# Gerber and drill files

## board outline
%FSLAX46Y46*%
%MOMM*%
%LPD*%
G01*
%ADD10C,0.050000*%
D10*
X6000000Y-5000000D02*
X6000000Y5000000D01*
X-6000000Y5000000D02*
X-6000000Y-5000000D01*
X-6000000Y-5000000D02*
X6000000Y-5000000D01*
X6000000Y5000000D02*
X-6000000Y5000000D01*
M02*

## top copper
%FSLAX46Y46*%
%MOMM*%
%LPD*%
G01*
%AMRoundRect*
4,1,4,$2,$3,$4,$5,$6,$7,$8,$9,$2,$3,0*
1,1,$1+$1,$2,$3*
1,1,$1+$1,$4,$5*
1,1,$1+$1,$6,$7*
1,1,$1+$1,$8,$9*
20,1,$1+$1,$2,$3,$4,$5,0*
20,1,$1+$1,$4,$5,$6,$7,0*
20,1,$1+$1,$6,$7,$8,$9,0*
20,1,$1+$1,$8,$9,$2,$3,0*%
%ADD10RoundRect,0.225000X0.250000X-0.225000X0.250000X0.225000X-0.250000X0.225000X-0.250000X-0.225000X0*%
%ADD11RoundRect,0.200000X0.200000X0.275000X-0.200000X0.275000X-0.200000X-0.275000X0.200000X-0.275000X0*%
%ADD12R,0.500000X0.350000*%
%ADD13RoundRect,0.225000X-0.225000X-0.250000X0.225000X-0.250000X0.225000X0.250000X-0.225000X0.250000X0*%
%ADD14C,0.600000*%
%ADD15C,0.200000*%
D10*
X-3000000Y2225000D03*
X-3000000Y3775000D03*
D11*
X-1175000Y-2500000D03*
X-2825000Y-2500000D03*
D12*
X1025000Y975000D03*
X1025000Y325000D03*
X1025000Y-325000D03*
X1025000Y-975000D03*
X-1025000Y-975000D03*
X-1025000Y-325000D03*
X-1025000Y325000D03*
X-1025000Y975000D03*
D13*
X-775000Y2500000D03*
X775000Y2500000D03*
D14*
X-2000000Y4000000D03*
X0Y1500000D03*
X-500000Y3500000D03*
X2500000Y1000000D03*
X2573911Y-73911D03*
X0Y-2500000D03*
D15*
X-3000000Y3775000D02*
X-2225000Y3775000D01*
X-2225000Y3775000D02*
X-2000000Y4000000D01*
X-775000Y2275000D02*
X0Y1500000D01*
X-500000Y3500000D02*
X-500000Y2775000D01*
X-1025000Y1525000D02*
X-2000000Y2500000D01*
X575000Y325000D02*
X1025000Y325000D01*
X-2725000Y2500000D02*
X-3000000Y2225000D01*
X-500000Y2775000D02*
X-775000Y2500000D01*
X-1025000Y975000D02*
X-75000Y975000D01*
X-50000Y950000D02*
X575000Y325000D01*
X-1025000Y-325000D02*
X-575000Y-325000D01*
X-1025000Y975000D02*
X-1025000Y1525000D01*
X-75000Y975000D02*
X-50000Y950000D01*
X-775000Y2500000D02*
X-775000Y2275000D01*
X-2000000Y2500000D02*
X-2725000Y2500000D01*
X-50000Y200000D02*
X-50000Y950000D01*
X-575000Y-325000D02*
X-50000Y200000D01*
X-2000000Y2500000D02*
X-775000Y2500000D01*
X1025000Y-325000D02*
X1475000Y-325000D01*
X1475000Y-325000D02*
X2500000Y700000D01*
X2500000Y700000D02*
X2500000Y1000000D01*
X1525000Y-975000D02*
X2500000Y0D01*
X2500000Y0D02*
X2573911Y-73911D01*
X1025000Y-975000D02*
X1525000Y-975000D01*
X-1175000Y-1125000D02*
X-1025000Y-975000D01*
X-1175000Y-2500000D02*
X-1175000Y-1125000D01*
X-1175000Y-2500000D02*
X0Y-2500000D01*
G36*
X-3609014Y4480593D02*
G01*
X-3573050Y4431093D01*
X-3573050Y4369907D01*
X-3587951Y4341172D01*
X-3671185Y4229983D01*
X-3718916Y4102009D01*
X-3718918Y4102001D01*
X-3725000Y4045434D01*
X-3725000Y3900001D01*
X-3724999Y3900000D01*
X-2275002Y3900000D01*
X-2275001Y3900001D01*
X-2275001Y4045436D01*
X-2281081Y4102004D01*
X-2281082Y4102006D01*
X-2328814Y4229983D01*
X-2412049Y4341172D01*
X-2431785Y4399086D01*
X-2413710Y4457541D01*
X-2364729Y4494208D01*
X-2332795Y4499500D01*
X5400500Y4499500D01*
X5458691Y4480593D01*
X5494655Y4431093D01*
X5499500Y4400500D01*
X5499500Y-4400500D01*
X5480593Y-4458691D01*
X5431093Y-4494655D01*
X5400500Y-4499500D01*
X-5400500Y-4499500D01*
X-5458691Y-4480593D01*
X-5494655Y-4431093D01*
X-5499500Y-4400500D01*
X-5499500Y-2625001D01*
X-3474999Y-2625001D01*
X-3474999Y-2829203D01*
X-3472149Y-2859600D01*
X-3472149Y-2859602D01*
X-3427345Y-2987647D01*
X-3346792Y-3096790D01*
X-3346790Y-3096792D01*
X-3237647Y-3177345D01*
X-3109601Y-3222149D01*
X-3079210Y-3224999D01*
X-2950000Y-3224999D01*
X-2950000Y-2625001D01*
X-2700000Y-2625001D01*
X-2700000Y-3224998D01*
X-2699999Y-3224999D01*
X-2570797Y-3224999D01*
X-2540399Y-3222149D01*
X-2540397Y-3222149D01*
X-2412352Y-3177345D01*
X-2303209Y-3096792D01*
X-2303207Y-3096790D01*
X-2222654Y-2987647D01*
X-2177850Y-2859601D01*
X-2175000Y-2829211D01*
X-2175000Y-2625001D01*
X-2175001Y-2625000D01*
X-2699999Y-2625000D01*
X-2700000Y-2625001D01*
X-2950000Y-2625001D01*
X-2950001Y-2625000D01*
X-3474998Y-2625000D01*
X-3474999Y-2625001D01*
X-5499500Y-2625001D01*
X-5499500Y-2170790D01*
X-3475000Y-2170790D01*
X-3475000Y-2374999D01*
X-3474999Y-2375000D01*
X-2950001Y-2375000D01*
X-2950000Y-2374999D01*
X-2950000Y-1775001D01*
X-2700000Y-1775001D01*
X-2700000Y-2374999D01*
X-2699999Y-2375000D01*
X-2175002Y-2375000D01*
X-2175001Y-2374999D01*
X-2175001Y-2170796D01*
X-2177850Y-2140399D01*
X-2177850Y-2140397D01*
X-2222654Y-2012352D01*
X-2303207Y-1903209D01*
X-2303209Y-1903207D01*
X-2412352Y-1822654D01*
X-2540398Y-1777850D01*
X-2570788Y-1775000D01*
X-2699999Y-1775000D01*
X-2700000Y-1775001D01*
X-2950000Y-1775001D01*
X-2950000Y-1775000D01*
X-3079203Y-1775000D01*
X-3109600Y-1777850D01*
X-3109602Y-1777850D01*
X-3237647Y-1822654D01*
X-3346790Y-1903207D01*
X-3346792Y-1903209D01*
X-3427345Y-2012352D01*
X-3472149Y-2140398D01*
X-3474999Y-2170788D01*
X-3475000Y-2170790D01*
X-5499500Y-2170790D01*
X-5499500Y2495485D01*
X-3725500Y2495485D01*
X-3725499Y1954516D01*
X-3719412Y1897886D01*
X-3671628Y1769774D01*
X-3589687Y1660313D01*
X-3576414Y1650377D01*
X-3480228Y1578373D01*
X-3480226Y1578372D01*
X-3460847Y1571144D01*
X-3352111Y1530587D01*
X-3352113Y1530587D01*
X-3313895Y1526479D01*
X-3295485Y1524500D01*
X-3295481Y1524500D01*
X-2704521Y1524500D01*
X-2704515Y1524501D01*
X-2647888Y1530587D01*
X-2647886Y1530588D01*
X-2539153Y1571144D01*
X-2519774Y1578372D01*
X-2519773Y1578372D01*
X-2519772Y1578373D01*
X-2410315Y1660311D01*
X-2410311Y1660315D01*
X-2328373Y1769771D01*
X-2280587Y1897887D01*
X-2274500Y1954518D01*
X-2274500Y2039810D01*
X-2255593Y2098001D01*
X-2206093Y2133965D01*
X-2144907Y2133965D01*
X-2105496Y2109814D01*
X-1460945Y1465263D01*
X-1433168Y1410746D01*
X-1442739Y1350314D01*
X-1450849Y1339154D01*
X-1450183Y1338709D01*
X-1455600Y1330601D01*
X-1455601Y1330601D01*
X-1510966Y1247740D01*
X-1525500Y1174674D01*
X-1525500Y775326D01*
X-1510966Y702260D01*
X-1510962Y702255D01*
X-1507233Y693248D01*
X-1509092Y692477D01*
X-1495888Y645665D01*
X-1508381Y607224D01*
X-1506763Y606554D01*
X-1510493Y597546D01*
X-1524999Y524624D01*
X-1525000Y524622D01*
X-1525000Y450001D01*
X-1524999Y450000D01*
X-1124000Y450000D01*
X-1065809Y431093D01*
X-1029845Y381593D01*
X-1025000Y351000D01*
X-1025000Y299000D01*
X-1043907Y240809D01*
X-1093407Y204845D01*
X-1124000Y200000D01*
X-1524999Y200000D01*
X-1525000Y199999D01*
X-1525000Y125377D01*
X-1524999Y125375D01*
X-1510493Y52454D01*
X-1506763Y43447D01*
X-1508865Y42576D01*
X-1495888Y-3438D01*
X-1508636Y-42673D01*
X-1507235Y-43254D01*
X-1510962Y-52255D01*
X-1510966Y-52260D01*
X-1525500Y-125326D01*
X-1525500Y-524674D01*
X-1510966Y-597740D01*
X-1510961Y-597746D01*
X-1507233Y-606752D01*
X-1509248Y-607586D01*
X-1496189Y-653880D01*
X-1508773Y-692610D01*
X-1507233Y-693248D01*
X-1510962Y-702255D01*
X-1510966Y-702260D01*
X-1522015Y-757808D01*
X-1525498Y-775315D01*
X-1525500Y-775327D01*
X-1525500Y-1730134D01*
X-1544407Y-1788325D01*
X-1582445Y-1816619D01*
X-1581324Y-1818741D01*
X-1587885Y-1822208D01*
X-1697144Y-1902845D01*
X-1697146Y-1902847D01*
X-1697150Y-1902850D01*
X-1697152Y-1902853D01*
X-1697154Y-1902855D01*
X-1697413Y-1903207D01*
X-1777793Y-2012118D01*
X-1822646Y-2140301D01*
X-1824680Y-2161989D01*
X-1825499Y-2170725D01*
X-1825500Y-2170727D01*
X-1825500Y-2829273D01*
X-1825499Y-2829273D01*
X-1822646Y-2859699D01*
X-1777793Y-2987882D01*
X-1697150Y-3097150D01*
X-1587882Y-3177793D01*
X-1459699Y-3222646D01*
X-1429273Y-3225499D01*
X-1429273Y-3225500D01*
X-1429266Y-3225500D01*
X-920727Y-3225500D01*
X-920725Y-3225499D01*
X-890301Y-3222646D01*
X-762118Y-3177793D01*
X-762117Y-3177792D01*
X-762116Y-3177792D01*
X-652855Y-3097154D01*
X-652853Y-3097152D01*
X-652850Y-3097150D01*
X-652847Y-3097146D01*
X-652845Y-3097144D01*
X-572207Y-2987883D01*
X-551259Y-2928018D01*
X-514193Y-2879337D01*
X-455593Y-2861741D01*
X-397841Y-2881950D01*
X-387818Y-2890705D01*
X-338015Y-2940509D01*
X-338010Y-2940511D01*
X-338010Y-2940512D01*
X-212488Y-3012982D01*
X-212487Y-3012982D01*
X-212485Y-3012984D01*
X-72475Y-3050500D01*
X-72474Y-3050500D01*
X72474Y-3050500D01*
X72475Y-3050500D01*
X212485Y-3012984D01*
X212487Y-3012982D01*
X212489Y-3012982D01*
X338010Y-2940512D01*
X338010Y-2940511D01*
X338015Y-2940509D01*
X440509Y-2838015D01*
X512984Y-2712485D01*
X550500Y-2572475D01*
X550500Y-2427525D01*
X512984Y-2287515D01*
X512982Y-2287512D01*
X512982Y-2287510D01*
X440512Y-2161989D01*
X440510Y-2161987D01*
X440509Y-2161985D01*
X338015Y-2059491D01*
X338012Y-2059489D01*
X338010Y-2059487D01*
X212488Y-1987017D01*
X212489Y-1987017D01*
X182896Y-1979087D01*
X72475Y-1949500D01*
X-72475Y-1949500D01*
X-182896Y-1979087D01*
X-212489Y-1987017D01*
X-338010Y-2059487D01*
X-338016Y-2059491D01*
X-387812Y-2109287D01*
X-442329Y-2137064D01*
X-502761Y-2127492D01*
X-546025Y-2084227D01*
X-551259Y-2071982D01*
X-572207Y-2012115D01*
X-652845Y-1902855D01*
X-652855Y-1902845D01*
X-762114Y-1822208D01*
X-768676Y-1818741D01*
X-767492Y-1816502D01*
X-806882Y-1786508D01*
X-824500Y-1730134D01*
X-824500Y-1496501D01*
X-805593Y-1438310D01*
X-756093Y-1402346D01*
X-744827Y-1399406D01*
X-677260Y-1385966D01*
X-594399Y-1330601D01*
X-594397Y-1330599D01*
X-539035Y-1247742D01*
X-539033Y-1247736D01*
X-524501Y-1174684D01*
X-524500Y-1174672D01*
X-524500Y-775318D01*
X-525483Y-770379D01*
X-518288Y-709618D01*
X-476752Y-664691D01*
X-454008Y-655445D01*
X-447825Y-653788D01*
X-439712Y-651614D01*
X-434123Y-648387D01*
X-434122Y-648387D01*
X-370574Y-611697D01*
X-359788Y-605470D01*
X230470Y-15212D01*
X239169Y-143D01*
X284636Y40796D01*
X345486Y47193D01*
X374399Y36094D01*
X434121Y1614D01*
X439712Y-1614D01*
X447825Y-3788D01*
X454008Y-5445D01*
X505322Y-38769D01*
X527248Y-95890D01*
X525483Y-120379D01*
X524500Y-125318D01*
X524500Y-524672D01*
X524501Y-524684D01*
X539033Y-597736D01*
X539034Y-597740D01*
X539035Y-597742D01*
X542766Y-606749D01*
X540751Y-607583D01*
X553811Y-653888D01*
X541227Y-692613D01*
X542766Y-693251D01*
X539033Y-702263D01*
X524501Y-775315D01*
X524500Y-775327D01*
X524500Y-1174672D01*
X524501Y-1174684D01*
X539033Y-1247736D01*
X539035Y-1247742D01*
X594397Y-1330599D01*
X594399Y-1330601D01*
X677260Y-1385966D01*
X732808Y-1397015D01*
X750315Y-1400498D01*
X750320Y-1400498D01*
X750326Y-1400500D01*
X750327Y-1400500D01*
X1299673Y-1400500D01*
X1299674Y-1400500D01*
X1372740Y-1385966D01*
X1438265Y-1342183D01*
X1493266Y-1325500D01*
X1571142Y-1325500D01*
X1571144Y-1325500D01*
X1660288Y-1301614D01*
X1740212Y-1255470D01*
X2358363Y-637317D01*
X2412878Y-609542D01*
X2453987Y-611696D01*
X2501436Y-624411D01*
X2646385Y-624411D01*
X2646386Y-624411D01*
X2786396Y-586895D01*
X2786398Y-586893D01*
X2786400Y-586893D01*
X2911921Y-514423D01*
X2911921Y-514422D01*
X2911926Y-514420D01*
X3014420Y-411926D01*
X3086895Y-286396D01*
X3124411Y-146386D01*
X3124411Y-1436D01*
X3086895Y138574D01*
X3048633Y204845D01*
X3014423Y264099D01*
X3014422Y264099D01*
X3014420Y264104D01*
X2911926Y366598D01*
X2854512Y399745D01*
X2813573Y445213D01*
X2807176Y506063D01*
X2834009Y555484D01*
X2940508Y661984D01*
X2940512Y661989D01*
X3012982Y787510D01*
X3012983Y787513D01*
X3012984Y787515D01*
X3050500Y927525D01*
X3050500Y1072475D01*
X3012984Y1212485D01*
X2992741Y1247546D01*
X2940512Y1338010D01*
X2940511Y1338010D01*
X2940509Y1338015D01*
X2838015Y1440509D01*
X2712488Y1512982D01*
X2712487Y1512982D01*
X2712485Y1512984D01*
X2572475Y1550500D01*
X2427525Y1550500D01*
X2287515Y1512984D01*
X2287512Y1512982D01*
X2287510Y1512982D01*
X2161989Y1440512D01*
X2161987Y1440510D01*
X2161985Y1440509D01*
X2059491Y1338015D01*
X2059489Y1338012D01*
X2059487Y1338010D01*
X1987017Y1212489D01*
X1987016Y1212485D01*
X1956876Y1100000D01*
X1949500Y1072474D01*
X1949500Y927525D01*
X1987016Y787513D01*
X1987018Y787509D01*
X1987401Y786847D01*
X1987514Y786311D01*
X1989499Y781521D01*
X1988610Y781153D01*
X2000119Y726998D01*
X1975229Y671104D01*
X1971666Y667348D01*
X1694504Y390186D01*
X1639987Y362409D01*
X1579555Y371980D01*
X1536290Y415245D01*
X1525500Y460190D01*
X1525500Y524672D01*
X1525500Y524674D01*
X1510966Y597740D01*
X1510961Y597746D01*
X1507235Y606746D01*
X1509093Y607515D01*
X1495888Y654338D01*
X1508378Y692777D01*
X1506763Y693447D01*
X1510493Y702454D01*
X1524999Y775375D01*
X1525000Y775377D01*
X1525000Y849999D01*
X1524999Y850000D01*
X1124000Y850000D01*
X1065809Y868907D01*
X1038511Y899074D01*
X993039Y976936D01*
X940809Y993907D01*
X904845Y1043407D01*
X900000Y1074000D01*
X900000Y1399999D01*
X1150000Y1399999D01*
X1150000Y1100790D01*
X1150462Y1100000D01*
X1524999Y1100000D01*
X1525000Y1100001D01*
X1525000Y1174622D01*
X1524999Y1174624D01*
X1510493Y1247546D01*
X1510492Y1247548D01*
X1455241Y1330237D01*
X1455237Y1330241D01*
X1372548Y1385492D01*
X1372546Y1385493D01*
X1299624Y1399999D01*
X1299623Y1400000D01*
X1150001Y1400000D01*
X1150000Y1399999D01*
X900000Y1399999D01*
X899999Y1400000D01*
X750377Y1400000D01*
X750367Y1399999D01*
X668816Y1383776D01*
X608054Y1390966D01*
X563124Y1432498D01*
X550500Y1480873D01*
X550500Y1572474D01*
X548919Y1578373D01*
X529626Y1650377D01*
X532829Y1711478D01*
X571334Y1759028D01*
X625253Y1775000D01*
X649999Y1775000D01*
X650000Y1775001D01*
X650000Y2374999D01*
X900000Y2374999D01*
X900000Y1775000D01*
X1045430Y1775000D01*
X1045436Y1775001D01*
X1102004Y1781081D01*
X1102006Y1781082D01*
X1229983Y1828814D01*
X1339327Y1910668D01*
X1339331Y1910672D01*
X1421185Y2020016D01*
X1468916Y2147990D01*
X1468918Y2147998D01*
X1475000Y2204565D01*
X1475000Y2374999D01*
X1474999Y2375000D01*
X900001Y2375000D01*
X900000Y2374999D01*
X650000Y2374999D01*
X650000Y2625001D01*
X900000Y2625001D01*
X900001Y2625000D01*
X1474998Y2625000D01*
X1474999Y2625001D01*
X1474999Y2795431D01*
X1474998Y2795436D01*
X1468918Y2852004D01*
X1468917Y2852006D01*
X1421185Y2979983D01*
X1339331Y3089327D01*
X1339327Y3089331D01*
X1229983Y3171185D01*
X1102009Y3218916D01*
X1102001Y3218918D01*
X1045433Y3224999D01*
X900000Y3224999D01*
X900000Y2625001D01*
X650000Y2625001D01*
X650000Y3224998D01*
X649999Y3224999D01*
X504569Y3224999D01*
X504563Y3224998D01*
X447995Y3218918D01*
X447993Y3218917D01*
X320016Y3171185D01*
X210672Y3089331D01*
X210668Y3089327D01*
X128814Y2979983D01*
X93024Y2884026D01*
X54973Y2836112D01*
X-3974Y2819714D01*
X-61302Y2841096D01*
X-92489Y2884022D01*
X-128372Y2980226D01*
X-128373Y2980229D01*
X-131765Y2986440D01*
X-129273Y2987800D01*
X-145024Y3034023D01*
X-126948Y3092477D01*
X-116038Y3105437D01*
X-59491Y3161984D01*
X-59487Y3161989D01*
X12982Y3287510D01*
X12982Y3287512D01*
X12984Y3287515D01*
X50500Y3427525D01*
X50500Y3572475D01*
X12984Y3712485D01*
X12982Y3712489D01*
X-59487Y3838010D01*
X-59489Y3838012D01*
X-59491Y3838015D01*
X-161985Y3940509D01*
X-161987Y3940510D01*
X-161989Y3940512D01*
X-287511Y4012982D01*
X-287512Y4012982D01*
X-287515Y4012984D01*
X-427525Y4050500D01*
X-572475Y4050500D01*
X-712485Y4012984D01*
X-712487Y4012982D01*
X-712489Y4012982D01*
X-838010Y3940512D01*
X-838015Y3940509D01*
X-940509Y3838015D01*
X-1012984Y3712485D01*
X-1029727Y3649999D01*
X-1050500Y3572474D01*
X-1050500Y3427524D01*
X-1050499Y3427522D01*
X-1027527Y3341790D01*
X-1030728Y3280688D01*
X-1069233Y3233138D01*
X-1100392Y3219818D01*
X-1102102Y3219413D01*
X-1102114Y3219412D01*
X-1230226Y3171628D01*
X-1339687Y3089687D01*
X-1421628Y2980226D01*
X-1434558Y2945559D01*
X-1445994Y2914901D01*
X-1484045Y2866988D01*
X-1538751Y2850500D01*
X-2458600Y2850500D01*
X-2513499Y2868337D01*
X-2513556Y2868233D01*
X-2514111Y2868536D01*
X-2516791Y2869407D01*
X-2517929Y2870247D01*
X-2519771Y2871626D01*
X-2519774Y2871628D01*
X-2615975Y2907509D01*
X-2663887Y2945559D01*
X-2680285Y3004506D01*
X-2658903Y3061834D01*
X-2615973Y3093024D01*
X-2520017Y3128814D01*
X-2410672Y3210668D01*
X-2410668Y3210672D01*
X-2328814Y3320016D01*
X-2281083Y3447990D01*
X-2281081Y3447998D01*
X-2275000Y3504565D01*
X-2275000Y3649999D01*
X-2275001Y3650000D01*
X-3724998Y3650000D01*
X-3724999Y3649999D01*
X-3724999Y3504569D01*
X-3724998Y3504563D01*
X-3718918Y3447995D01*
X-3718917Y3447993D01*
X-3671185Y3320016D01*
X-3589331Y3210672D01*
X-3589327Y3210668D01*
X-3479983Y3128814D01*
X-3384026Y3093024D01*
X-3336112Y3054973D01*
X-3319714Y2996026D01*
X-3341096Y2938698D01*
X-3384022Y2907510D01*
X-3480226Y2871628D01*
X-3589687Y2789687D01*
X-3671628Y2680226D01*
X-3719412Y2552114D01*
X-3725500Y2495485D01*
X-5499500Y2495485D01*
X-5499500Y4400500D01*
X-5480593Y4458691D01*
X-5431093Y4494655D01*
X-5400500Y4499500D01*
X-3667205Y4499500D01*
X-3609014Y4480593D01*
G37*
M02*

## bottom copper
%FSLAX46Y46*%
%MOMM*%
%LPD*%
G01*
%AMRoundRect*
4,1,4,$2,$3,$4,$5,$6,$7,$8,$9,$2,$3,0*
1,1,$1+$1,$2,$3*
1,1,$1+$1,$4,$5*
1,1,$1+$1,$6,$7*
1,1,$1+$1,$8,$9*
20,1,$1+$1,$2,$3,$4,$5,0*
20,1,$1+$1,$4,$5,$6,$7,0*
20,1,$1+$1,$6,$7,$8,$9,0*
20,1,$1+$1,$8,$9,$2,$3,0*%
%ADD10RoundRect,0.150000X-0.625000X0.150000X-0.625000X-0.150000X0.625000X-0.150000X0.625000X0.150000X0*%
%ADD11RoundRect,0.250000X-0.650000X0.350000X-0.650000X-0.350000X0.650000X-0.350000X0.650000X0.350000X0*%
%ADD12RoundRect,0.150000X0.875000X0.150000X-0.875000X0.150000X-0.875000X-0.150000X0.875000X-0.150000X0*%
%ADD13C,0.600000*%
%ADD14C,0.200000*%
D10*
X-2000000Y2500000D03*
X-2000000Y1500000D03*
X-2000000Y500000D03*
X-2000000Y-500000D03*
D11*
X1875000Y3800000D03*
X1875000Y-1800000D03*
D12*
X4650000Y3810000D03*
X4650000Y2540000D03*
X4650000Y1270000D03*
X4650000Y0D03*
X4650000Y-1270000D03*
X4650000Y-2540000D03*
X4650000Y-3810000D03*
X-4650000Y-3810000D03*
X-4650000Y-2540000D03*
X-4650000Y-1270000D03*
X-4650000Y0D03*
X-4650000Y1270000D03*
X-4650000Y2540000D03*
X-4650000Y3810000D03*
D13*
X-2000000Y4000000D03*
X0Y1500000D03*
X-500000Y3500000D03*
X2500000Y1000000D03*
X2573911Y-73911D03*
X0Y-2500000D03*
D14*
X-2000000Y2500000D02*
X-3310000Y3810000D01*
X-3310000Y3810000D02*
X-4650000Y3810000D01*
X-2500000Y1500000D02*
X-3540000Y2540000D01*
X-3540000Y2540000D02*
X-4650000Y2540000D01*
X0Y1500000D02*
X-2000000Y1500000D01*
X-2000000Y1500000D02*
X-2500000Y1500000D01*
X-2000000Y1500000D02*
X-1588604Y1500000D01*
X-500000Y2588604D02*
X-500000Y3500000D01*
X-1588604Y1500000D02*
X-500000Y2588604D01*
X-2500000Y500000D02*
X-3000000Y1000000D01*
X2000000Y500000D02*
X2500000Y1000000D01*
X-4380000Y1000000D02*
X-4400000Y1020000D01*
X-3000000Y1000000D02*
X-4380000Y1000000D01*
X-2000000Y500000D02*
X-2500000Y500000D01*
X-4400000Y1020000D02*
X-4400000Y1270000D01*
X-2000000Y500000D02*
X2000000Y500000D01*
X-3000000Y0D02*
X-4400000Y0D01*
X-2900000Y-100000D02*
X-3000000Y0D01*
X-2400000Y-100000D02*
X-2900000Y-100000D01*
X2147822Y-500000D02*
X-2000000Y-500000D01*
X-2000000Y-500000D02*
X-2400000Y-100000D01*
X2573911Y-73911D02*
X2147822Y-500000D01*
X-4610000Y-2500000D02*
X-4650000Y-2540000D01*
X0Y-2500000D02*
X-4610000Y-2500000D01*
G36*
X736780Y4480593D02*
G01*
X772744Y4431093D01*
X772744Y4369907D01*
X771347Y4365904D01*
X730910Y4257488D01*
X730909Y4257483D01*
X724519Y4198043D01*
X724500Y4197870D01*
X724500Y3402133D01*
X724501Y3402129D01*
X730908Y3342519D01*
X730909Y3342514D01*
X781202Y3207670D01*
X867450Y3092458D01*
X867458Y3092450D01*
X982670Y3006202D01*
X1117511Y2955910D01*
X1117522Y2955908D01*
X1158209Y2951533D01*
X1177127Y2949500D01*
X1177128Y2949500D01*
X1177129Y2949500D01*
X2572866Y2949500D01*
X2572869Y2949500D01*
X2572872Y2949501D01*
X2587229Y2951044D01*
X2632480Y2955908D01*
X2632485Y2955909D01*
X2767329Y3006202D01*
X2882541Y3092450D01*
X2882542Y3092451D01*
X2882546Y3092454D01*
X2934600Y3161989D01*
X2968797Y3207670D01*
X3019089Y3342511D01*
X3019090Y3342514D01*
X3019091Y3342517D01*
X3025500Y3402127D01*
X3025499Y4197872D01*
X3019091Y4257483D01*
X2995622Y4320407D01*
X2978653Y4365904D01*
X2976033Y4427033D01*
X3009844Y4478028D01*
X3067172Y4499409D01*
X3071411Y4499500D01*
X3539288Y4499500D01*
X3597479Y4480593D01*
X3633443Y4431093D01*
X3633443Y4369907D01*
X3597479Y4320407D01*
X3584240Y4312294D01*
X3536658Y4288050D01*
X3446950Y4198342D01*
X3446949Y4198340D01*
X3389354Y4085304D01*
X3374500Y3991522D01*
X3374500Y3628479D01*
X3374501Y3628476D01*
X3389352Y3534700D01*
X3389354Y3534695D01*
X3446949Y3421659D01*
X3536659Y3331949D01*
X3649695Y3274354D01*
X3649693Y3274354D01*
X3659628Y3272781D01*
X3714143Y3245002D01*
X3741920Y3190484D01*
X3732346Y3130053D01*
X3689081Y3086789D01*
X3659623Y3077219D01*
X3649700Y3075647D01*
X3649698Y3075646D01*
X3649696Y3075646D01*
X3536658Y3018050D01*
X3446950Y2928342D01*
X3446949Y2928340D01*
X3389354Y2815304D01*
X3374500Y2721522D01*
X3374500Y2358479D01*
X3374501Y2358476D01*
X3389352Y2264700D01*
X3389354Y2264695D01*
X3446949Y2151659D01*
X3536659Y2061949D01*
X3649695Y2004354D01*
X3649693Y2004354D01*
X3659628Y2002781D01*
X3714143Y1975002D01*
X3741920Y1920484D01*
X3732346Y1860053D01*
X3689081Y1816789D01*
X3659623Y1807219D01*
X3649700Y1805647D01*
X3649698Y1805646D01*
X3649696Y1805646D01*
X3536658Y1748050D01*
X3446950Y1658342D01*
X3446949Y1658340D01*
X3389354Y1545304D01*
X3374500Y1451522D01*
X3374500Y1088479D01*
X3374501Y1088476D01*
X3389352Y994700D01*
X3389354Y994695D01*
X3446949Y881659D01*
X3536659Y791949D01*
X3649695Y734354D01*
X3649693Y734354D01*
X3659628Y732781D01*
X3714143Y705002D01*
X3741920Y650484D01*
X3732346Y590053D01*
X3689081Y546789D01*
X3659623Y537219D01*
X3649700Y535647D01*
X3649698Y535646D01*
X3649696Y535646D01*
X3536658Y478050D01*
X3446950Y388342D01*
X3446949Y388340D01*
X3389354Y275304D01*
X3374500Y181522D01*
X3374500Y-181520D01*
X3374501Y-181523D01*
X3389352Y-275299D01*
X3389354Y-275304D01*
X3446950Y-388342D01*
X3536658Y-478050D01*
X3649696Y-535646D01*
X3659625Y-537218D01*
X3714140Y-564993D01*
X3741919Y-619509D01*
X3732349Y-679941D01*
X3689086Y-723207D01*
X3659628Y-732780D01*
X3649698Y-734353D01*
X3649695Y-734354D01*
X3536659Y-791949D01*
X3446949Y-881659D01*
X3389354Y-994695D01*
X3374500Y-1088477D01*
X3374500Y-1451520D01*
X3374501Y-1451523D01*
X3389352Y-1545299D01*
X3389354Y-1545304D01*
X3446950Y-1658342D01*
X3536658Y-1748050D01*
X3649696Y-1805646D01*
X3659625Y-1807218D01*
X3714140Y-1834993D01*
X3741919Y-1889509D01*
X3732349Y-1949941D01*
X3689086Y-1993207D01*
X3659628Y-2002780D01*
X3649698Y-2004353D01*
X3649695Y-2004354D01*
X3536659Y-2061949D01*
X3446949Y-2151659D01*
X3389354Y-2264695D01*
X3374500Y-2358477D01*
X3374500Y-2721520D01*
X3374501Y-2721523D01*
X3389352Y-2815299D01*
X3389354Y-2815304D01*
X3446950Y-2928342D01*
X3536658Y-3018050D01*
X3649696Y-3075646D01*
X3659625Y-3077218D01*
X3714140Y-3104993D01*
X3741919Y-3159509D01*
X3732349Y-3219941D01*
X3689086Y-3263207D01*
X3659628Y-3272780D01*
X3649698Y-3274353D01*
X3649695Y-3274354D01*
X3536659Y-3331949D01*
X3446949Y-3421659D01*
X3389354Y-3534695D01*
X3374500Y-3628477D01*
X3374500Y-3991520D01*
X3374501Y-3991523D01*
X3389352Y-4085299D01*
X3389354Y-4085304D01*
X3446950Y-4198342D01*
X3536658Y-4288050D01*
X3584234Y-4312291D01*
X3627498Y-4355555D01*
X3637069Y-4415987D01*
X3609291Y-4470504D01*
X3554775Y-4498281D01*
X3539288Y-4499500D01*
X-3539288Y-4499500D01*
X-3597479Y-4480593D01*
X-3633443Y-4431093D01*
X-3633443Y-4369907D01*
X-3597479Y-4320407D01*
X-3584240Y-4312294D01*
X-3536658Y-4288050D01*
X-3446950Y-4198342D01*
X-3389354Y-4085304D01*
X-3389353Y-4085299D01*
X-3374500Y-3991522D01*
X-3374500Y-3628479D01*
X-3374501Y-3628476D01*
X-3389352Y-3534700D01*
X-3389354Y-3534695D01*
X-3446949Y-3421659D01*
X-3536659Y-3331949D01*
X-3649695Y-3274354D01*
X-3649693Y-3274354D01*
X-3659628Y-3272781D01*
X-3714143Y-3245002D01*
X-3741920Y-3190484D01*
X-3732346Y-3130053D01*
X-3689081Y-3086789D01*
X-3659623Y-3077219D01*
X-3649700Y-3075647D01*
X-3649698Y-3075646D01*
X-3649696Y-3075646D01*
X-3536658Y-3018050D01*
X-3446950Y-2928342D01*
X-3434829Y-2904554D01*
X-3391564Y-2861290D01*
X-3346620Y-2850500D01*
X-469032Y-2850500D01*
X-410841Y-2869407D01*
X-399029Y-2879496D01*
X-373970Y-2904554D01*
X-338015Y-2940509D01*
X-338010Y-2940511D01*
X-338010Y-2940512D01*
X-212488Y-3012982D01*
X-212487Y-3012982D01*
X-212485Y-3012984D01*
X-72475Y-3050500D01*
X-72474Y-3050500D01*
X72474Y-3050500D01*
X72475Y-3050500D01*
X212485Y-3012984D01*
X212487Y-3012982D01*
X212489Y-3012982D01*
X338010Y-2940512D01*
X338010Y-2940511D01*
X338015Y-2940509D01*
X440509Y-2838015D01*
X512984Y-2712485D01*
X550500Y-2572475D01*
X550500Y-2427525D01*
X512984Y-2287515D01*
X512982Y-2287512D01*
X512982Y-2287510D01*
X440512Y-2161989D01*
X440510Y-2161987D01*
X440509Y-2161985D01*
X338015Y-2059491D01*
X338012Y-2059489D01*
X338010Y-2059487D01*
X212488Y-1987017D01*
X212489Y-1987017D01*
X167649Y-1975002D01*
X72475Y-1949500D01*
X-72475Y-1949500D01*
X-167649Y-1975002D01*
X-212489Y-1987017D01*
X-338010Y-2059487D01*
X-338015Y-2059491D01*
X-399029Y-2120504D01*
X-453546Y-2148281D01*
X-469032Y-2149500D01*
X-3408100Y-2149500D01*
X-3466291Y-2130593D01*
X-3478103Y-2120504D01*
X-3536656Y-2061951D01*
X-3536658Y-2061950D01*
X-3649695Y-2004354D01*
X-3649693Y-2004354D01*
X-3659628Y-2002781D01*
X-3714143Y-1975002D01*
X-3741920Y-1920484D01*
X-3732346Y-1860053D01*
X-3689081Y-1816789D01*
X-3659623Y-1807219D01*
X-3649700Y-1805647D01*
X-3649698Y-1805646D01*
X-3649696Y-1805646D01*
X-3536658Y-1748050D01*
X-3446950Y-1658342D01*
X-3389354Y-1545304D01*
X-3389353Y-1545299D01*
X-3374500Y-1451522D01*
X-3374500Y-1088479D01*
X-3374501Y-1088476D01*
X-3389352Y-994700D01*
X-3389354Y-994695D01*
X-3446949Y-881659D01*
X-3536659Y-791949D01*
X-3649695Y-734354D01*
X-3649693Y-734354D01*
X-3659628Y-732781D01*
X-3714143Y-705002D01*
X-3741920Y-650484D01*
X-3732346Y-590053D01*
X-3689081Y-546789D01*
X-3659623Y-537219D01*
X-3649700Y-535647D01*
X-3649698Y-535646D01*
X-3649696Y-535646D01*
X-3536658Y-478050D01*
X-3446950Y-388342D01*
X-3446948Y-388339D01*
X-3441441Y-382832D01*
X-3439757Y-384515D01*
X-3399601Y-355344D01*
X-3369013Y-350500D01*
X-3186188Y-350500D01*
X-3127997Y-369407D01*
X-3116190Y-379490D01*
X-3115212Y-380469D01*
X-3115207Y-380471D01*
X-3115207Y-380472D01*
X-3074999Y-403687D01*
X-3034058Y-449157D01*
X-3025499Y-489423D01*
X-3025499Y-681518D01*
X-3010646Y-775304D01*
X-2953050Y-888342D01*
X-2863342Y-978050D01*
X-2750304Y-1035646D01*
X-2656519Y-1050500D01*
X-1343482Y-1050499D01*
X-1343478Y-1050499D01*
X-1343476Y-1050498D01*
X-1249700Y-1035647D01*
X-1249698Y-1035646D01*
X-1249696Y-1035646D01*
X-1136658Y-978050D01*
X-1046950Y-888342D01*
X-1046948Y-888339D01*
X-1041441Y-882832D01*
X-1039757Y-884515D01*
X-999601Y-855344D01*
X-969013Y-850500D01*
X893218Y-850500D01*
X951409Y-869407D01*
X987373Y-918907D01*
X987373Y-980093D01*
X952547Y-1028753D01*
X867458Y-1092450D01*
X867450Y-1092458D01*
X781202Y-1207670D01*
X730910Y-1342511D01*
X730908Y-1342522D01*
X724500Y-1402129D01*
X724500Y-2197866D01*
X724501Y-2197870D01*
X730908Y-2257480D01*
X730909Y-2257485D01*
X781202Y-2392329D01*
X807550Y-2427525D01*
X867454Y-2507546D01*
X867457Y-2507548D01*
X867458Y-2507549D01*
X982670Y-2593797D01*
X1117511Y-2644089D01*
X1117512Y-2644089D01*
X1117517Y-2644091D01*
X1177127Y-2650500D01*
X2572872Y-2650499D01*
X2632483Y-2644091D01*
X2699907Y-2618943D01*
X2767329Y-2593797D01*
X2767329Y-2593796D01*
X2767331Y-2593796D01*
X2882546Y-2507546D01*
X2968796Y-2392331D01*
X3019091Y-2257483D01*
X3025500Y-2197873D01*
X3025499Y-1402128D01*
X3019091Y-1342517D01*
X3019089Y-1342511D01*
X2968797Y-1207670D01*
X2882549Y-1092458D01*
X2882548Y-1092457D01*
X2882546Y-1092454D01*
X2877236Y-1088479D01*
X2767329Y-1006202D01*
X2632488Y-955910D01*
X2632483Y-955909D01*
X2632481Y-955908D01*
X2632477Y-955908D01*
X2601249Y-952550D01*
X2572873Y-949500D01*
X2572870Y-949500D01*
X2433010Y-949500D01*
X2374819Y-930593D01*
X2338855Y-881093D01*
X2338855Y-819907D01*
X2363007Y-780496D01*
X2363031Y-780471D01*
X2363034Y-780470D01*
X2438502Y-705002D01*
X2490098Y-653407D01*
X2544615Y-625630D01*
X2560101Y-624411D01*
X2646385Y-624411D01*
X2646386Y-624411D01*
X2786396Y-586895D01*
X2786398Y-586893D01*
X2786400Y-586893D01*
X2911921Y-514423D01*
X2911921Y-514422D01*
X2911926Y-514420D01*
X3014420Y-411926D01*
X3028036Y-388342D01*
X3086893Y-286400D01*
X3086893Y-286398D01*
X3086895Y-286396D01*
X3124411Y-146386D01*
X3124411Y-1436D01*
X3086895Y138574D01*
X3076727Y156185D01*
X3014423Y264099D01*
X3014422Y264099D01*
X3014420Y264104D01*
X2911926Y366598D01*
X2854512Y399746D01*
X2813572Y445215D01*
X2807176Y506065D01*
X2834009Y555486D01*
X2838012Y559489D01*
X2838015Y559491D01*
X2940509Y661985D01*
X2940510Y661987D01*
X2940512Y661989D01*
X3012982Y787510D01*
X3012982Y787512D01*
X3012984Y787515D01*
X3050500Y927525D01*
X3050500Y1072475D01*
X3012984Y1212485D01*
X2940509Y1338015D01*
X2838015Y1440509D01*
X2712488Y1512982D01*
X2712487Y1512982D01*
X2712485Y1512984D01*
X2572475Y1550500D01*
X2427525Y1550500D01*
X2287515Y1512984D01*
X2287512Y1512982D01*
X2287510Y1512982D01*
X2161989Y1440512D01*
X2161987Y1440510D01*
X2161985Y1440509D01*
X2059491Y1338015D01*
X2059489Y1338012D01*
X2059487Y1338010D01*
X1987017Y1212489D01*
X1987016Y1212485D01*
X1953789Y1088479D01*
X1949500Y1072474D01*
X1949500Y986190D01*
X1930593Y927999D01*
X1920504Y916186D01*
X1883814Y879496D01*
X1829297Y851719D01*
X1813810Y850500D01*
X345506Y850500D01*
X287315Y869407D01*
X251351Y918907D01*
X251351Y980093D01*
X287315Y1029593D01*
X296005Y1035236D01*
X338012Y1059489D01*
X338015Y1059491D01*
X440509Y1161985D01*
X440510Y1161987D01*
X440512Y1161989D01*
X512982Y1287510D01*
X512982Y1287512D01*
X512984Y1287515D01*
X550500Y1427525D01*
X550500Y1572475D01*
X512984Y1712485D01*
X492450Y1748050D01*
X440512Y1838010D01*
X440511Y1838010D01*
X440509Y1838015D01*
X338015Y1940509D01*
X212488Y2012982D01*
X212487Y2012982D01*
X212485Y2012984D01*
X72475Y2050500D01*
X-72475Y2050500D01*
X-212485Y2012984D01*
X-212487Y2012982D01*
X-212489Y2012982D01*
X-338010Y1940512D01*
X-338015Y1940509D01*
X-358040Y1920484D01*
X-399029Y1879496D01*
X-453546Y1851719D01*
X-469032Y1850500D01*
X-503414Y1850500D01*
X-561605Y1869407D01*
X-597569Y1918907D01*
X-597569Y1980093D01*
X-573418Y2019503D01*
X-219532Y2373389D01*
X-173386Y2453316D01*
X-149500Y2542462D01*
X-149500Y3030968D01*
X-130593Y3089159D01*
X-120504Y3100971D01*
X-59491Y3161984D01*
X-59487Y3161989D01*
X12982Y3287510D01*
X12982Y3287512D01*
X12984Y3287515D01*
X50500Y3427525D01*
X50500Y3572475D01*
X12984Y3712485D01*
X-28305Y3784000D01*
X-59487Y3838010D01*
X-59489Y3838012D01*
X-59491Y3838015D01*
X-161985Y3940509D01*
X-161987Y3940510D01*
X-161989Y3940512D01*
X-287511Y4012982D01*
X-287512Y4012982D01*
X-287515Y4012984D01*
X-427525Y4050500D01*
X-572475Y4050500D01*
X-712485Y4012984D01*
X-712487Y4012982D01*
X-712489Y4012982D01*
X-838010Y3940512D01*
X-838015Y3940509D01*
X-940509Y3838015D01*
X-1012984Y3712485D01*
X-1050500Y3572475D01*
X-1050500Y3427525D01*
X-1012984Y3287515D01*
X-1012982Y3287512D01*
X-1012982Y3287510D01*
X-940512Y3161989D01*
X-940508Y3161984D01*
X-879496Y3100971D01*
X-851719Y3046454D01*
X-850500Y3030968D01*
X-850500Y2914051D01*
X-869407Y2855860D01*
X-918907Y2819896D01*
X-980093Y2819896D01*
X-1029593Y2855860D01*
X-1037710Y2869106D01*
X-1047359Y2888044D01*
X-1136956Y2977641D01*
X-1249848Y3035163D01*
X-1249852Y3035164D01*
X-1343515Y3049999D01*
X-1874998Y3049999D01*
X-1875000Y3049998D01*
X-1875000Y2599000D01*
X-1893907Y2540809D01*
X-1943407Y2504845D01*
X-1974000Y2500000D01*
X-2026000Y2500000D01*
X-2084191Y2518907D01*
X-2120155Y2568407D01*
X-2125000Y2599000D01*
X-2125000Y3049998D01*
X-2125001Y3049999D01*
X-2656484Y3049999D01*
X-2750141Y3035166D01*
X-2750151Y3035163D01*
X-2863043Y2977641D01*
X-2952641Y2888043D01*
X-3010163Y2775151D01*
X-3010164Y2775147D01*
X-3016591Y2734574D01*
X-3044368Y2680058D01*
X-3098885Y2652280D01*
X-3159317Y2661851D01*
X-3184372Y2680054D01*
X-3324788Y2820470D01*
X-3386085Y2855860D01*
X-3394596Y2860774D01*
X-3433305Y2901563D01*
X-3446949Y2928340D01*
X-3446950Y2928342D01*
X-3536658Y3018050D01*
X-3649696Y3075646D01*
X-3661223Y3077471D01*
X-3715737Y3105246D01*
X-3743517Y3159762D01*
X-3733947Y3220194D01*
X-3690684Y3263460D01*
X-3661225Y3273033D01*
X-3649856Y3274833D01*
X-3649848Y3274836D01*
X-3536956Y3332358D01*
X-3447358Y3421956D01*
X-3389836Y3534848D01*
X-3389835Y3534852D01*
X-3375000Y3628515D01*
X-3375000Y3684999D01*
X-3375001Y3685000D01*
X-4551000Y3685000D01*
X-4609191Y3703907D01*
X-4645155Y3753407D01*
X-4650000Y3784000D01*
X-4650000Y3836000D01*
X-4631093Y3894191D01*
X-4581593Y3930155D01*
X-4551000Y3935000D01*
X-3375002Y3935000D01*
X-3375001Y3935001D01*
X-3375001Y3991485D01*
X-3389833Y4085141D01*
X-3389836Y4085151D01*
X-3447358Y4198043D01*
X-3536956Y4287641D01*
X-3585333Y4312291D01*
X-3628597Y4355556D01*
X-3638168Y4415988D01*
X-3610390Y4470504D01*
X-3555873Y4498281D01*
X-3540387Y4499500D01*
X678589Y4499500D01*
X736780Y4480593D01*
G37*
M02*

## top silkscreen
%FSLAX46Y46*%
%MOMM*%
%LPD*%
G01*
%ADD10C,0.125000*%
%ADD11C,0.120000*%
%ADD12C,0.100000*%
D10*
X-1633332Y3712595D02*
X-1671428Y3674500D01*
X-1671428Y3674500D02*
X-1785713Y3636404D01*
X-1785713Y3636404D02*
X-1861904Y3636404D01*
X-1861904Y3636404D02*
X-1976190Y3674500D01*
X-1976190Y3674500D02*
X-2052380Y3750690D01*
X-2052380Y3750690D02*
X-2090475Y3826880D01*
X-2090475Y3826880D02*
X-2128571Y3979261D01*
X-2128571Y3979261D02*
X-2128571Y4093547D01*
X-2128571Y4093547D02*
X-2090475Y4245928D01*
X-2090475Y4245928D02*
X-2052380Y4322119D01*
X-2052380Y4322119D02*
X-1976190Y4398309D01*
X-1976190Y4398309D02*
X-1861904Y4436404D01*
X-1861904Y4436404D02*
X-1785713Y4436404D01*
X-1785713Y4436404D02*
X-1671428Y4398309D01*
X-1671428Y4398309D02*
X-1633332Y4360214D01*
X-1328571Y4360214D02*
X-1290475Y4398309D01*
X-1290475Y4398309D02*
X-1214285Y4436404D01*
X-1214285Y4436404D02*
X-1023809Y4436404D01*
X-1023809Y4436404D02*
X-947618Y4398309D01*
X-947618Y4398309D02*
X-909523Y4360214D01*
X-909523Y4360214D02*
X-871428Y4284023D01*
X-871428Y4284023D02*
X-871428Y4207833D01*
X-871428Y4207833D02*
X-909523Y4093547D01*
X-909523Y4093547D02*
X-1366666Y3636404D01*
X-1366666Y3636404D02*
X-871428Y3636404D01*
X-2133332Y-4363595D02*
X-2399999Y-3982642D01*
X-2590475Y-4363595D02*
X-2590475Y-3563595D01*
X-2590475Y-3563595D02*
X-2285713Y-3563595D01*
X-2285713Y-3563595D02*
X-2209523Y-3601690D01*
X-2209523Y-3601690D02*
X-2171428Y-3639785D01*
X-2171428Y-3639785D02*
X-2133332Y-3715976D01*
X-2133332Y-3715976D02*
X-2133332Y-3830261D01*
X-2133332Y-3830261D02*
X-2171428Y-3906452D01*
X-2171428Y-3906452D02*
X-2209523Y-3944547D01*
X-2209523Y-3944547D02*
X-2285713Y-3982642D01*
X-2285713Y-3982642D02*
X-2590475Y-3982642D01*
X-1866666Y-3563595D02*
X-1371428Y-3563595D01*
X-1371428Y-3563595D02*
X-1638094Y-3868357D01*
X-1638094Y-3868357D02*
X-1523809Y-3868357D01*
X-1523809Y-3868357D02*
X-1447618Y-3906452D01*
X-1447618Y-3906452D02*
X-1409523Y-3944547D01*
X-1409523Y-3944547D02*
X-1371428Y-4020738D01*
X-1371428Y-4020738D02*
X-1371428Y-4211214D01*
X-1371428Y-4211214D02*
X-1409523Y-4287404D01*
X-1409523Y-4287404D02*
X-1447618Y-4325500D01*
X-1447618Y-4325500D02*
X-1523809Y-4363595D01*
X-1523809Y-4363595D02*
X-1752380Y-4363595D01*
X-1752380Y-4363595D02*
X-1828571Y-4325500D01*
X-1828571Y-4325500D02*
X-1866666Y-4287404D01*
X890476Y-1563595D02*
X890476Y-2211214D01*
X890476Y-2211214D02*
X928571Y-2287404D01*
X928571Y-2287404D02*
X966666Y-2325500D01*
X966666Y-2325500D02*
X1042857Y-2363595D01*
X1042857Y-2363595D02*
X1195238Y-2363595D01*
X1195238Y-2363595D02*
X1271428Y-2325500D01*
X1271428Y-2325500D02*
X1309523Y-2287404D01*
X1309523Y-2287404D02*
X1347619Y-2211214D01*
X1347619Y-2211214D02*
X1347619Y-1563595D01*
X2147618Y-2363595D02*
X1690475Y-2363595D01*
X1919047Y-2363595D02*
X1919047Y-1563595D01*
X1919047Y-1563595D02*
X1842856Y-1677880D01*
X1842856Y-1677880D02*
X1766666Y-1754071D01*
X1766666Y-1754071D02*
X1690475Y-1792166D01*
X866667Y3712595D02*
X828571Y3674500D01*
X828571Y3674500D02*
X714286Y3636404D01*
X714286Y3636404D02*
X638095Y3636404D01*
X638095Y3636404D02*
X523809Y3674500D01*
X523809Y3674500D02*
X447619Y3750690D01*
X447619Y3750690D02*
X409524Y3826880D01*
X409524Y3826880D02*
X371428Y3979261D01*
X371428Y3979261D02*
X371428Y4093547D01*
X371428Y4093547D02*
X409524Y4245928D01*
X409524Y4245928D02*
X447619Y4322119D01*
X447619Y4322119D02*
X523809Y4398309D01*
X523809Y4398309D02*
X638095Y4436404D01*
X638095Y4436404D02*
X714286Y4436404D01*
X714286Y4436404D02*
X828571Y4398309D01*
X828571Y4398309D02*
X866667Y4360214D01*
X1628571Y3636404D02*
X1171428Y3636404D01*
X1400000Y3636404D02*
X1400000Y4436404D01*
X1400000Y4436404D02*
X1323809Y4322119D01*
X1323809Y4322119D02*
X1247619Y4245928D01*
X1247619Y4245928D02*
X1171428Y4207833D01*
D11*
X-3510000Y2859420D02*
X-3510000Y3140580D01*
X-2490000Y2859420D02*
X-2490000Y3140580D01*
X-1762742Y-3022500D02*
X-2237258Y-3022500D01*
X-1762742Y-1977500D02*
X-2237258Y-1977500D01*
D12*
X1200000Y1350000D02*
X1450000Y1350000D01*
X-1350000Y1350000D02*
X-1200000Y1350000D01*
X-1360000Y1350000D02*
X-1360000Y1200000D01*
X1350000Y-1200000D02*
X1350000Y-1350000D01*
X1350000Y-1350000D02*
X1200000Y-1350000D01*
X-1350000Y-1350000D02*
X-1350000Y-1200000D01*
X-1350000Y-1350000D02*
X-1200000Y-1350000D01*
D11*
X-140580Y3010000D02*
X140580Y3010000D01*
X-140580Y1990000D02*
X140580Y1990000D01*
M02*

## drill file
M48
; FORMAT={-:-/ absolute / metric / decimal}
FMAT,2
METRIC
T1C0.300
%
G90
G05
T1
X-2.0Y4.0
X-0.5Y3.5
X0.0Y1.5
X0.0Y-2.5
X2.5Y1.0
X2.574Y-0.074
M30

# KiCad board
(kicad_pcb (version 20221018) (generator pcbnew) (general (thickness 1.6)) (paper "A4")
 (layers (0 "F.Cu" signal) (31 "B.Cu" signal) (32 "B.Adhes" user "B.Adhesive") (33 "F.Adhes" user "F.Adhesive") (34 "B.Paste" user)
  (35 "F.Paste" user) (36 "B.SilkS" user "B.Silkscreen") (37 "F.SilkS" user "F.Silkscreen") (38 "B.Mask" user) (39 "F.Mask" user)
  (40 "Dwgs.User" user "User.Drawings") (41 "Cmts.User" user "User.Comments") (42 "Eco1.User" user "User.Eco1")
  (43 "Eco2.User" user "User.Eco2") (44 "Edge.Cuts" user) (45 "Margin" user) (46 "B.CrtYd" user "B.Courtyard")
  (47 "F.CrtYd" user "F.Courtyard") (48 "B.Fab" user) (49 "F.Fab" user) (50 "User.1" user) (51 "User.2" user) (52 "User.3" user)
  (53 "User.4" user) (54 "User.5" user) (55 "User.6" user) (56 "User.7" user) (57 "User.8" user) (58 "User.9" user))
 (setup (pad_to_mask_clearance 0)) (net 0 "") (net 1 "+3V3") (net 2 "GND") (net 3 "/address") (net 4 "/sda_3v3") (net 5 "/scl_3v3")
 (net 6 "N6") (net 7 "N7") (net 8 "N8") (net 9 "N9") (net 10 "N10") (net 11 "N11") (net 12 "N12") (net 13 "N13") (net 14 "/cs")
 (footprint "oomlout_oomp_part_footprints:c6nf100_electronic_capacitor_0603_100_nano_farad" (layer "F.Cu") (at -3 -3 90)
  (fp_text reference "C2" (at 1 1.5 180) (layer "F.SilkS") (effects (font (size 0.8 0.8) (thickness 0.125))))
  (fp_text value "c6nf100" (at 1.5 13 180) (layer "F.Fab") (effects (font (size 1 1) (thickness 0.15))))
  (fp_line (start -0.14058 -0.51) (end 0.14058 -0.51) (stroke (width 0.12) (type solid)) (layer "F.SilkS"))
  (fp_line (start -0.14058 0.51) (end 0.14058 0.51) (stroke (width 0.12) (type solid)) (layer "F.SilkS"))
  (pad "1" smd roundrect (at -0.775 0 90) (size 0.9 0.95) (layers "F.Cu" "F.Paste" "F.Mask") (roundrect_rratio 0.25) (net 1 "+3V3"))
  (pad "2" smd roundrect (at 0.775 0 90) (size 0.9 0.95) (layers "F.Cu" "F.Paste" "F.Mask") (roundrect_rratio 0.25) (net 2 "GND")))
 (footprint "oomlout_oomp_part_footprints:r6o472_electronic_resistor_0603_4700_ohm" (layer "F.Cu") (at -2 2.5 180)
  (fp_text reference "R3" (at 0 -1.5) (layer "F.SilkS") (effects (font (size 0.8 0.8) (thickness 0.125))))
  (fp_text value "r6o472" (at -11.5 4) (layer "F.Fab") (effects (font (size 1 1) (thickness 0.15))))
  (fp_line (start -0.237258 -0.5225) (end 0.237258 -0.5225) (stroke (width 0.12) (type solid)) (layer "F.SilkS"))
  (fp_line (start -0.237258 0.5225) (end 0.237258 0.5225) (stroke (width 0.12) (type solid)) (layer "F.SilkS"))
  (pad "1" smd roundrect (at -0.825 0 180) (size 0.8 0.95) (layers "F.Cu" "F.Paste" "F.Mask") (roundrect_rratio 0.25) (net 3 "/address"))
  (pad "2" smd roundrect (at 0.825 0 180) (size 0.8 0.95) (layers "F.Cu" "F.Paste" "F.Mask") (roundrect_rratio 0.25) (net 2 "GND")))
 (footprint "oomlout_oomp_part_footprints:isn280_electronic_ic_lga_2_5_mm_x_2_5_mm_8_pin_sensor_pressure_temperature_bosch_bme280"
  (layer "F.Cu") (at 0 0 -90)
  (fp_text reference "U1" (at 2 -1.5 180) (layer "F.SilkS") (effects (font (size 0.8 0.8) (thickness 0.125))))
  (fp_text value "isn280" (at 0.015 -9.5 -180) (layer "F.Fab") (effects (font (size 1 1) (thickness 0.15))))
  (fp_line (start -1.35 -1.2) (end -1.35 -1.45) (stroke (width 0.1) (type solid)) (layer "F.SilkS"))
  (fp_line (start -1.35 1.35) (end -1.35 1.2) (stroke (width 0.1) (type solid)) (layer "F.SilkS"))
  (fp_line (start -1.35 1.36) (end -1.2 1.36) (stroke (width 0.1) (type solid)) (layer "F.SilkS"))
  (fp_line (start 1.2 -1.35) (end 1.35 -1.35) (stroke (width 0.1) (type solid)) (layer "F.SilkS"))
  (fp_line (start 1.35 -1.35) (end 1.35 -1.2) (stroke (width 0.1) (type solid)) (layer "F.SilkS"))
  (fp_line (start 1.35 1.35) (end 1.2 1.35) (stroke (width 0.1) (type solid)) (layer "F.SilkS"))
  (fp_line (start 1.35 1.35) (end 1.35 1.2) (stroke (width 0.1) (type solid)) (layer "F.SilkS"))
  (pad "1" smd rect (at -0.975 -1.025) (size 0.5 0.35) (layers "F.Cu" "F.Paste" "F.Mask") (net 2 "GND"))
  (pad "2" smd rect (at -0.325 -1.025) (size 0.5 0.35) (layers "F.Cu" "F.Paste" "F.Mask") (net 1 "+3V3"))
  (pad "3" smd rect (at 0.325 -1.025) (size 0.5 0.35) (layers "F.Cu" "F.Paste" "F.Mask") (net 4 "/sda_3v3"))
  (pad "4" smd rect (at 0.975 -1.025) (size 0.5 0.35) (layers "F.Cu" "F.Paste" "F.Mask") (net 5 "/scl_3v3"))
  (pad "5" smd rect (at 0.975 1.025) (size 0.5 0.35) (layers "F.Cu" "F.Paste" "F.Mask") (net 3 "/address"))
  (pad "6" smd rect (at 0.325 1.025) (size 0.5 0.35) (layers "F.Cu" "F.Paste" "F.Mask") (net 1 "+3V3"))
  (pad "7" smd rect (at -0.325 1.025) (size 0.5 0.35) (layers "F.Cu" "F.Paste" "F.Mask") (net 2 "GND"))
  (pad "8" smd rect (at -0.975 1.025) (size 0.5 0.35) (layers "F.Cu" "F.Paste" "F.Mask") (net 1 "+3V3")))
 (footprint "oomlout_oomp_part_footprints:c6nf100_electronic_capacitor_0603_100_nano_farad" (layer "F.Cu") (at 0 -2.5)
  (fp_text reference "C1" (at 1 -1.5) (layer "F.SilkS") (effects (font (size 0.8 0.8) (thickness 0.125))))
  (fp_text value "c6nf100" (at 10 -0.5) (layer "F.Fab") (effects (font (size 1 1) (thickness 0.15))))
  (fp_line (start -0.14058 -0.51) (end 0.14058 -0.51) (stroke (width 0.12) (type solid)) (layer "F.SilkS"))
  (fp_line (start -0.14058 0.51) (end 0.14058 0.51) (stroke (width 0.12) (type solid)) (layer "F.SilkS"))
  (pad "1" smd roundrect (at -0.775 0) (size 0.9 0.95) (layers "F.Cu" "F.Paste" "F.Mask") (roundrect_rratio 0.25) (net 1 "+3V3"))
  (pad "2" smd roundrect (at 0.775 0) (size 0.9 0.95) (layers "F.Cu" "F.Paste" "F.Mask") (roundrect_rratio 0.25) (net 2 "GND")))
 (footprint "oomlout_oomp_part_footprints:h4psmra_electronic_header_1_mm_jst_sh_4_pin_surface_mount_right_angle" (layer "B.Cu")
  (at 0 -1 -90)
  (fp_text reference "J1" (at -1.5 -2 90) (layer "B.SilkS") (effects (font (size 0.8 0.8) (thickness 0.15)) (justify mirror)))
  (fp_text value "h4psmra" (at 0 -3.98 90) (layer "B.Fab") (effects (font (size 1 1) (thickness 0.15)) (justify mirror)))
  (pad "1" smd roundrect (at -1.5 2 270) (size 0.6 1.55) (layers "B.Cu" "B.Paste" "B.Mask") (roundrect_rratio 0.25) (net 2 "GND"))
  (pad "2" smd roundrect (at -0.5 2 270) (size 0.6 1.55) (layers "B.Cu" "B.Paste" "B.Mask") (roundrect_rratio 0.25) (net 1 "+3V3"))
  (pad "3" smd roundrect (at 0.5 2 270) (size 0.6 1.55) (layers "B.Cu" "B.Paste" "B.Mask") (roundrect_rratio 0.25) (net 4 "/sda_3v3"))
  (pad "4" smd roundrect (at 1.5 2 270) (size 0.6 1.55) (layers "B.Cu" "B.Paste" "B.Mask") (roundrect_rratio 0.25) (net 5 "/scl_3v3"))
  (pad "MP" smd roundrect (at -2.8 -1.875 270) (size 1.2 1.8) (layers "B.Cu" "B.Paste" "B.Mask") (roundrect_rratio 0.2083333333))
  (pad "MP" smd roundrect (at 2.8 -1.875 270) (size 1.2 1.8) (layers "B.Cu" "B.Paste" "B.Mask") (roundrect_rratio 0.2083333333)))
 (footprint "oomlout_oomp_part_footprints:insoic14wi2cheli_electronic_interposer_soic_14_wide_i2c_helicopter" (layer "B.Cu") (at 0 0 180)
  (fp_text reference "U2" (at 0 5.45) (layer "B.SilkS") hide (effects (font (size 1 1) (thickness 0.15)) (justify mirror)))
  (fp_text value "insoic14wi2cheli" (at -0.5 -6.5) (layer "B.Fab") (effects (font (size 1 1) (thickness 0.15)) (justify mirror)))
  (pad "1" smd roundrect (at -4.65 3.81 180) (size 2.05 0.6) (layers "B.Cu" "B.Paste" "B.Mask") (roundrect_rratio 0.25) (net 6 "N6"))
  (pad "2" smd roundrect (at -4.65 2.54 180) (size 2.05 0.6) (layers "B.Cu" "B.Paste" "B.Mask") (roundrect_rratio 0.25) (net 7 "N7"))
  (pad "3" smd roundrect (at -4.65 1.27 180) (size 2.05 0.6) (layers "B.Cu" "B.Paste" "B.Mask") (roundrect_rratio 0.25) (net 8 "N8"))
  (pad "4" smd roundrect (at -4.65 0 180) (size 2.05 0.6) (layers "B.Cu" "B.Paste" "B.Mask") (roundrect_rratio 0.25) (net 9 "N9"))
  (pad "5" smd roundrect (at -4.65 -1.27 180) (size 2.05 0.6) (layers "B.Cu" "B.Paste" "B.Mask") (roundrect_rratio 0.25) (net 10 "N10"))
  (pad "6" smd roundrect (at -4.65 -2.54 180) (size 2.05 0.6) (layers "B.Cu" "B.Paste" "B.Mask") (roundrect_rratio 0.25) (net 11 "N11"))
  (pad "7" smd roundrect (at -4.65 -3.81 180) (size 2.05 0.6) (layers "B.Cu" "B.Paste" "B.Mask") (roundrect_rratio 0.25) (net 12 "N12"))
  (pad "8" smd roundrect (at 4.65 -3.81 180) (size 2.05 0.6) (layers "B.Cu" "B.Paste" "B.Mask") (roundrect_rratio 0.25) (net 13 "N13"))
  (pad "9" smd roundrect (at 4.65 -2.54 180) (size 2.05 0.6) (layers "B.Cu" "B.Paste" "B.Mask") (roundrect_rratio 0.25) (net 3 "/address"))
  (pad "10" smd roundrect (at 4.65 -1.27 180) (size 2.05 0.6) (layers "B.Cu" "B.Paste" "B.Mask") (roundrect_rratio 0.25) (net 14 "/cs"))
  (pad "11" smd roundrect (at 4.65 0 180) (size 2.05 0.6) (layers "B.Cu" "B.Paste" "B.Mask") (roundrect_rratio 0.25) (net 5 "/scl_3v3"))
  (pad "12" smd roundrect (at 4.65 1.27 180) (size 2.05 0.6) (layers "B.Cu" "B.Paste" "B.Mask") (roundrect_rratio 0.25) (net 4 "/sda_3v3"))
  (pad "13" smd roundrect (at 4.65 2.54 180) (size 2.05 0.6) (layers "B.Cu" "B.Paste" "B.Mask") (roundrect_rratio 0.25) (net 1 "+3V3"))
  (pad "14" smd roundrect (at 4.65 3.81 180) (size 2.05 0.6) (layers "B.Cu" "B.Paste" "B.Mask") (roundrect_rratio 0.25) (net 2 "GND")))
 (gr_line (start 6 5) (end 6 -5) (stroke (width 0.05) (type default)) (layer "Edge.Cuts"))
 (gr_line (start -6 -5) (end -6 5) (stroke (width 0.05) (type default)) (layer "Edge.Cuts"))
 (gr_line (start -6 5) (end 6 5) (stroke (width 0.05) (type default)) (layer "Edge.Cuts"))
 (gr_line (start 6 -5) (end -6 -5) (stroke (width 0.05) (type default)) (layer "Edge.Cuts"))
 (segment (start -3 -3.775) (end -2.225 -3.775) (width 0.2) (layer "F.Cu") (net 2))
 (segment (start -2.225 -3.775) (end -2 -4) (width 0.2) (layer "F.Cu") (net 2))
 (via (at -2 -4) (size 0.6) (drill 0.3) (layers "F.Cu" "B.Cu") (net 2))
 (segment (start -2 -2.5) (end -3.31 -3.81) (width 0.2) (layer "B.Cu") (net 2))
 (segment (start -3.31 -3.81) (end -4.65 -3.81) (width 0.2) (layer "B.Cu") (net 2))
 (segment (start -0.775 -2.275) (end 0 -1.5) (width 0.2) (layer "F.Cu") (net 1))
 (segment (start -0.5 -3.5) (end -0.5 -2.775) (width 0.2) (layer "F.Cu") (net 1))
 (segment (start -1.025 -1.525) (end -2 -2.5) (width 0.2) (layer "F.Cu") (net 1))
 (segment (start 0.575 -0.325) (end 1.025 -0.325) (width 0.2) (layer "F.Cu") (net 1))
 (segment (start -2.725 -2.5) (end -3 -2.225) (width 0.2) (layer "F.Cu") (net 1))
 (segment (start -0.5 -2.775) (end -0.775 -2.5) (width 0.2) (layer "F.Cu") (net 1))
 (segment (start -1.025 -0.975) (end -0.075 -0.975) (width 0.2) (layer "F.Cu") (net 1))
 (segment (start -0.05 -0.95) (end 0.575 -0.325) (width 0.2) (layer "F.Cu") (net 1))
 (segment (start -1.025 0.325) (end -0.575 0.325) (width 0.2) (layer "F.Cu") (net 1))
 (segment (start -1.025 -0.975) (end -1.025 -1.525) (width 0.2) (layer "F.Cu") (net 1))
 (segment (start -0.075 -0.975) (end -0.05 -0.95) (width 0.2) (layer "F.Cu") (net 1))
 (segment (start -0.775 -2.5) (end -0.775 -2.275) (width 0.2) (layer "F.Cu") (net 1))
 (segment (start -2 -2.5) (end -2.725 -2.5) (width 0.2) (layer "F.Cu") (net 1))
 (segment (start -0.05 -0.2) (end -0.05 -0.95) (width 0.2) (layer "F.Cu") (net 1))
 (segment (start -0.575 0.325) (end -0.05 -0.2) (width 0.2) (layer "F.Cu") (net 1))
 (segment (start -2 -2.5) (end -0.775 -2.5) (width 0.2) (layer "F.Cu") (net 1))
 (via (at 0 -1.5) (size 0.6) (drill 0.3) (layers "F.Cu" "B.Cu") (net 1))
 (via (at -0.5 -3.5) (size 0.6) (drill 0.3) (layers "F.Cu" "B.Cu") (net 1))
 (segment (start -2.5 -1.5) (end -3.54 -2.54) (width 0.2) (layer "B.Cu") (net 1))
 (segment (start -3.54 -2.54) (end -4.65 -2.54) (width 0.2) (layer "B.Cu") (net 1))
 (segment (start 0 -1.5) (end -2 -1.5) (width 0.2) (layer "B.Cu") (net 1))
 (segment (start -2 -1.5) (end -2.5 -1.5) (width 0.2) (layer "B.Cu") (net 1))
 (segment (start -2 -1.5) (end -1.588604 -1.5) (width 0.2) (layer "B.Cu") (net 1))
 (segment (start -0.5 -2.588604) (end -0.5 -3.5) (width 0.2) (layer "B.Cu") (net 1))
 (segment (start -1.588604 -1.5) (end -0.5 -2.588604) (width 0.2) (layer "B.Cu") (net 1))
 (segment (start 1.025 0.325) (end 1.475 0.325) (width 0.2) (layer "F.Cu") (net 4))
 (segment (start 1.475 0.325) (end 2.5 -0.7) (width 0.2) (layer "F.Cu") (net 4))
 (segment (start 2.5 -0.7) (end 2.5 -1) (width 0.2) (layer "F.Cu") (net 4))
 (via (at 2.5 -1) (size 0.6) (drill 0.3) (layers "F.Cu" "B.Cu") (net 4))
 (segment (start -2.5 -0.5) (end -3 -1) (width 0.2) (layer "B.Cu") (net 4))
 (segment (start 2 -0.5) (end 2.5 -1) (width 0.2) (layer "B.Cu") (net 4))
 (segment (start -4.38 -1) (end -4.4 -1.02) (width 0.2) (layer "B.Cu") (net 4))
 (segment (start -3 -1) (end -4.38 -1) (width 0.2) (layer "B.Cu") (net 4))
 (segment (start -2 -0.5) (end -2.5 -0.5) (width 0.2) (layer "B.Cu") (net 4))
 (segment (start -4.4 -1.02) (end -4.4 -1.27) (width 0.2) (layer "B.Cu") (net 4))
 (segment (start -2 -0.5) (end 2 -0.5) (width 0.2) (layer "B.Cu") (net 4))
 (segment (start 1.525 0.975) (end 2.5 0) (width 0.2) (layer "F.Cu") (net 5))
 (segment (start 2.5 0) (end 2.573911 0.073911) (width 0.2) (layer "F.Cu") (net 5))
 (segment (start 1.025 0.975) (end 1.525 0.975) (width 0.2) (layer "F.Cu") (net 5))
 (via (at 2.573911 0.073911) (size 0.6) (drill 0.3) (layers "F.Cu" "B.Cu") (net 5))
 (segment (start -3 0) (end -4.4 0) (width 0.2) (layer "B.Cu") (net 5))
 (segment (start -2.9 0.1) (end -3 0) (width 0.2) (layer "B.Cu") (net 5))
 (segment (start -2.4 0.1) (end -2.9 0.1) (width 0.2) (layer "B.Cu") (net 5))
 (segment (start 2.147822 0.5) (end -2 0.5) (width 0.2) (layer "B.Cu") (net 5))
 (segment (start -2 0.5) (end -2.4 0.1) (width 0.2) (layer "B.Cu") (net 5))
 (segment (start 2.573911 0.073911) (end 2.147822 0.5) (width 0.2) (layer "B.Cu") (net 5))
 (segment (start -1.175 1.125) (end -1.025 0.975) (width 0.2) (layer "F.Cu") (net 3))
 (segment (start -1.175 2.5) (end -1.175 1.125) (width 0.2) (layer "F.Cu") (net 3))
 (segment (start -1.175 2.5) (end 0 2.5) (width 0.2) (layer "F.Cu") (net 3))
 (via (at 0 2.5) (size 0.6) (drill 0.3) (layers "F.Cu" "B.Cu") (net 3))
 (segment (start -4.61 2.5) (end -4.65 2.54) (width 0.2) (layer "B.Cu") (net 3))
 (segment (start 0 2.5) (end -4.61 2.5) (width 0.2) (layer "B.Cu") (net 3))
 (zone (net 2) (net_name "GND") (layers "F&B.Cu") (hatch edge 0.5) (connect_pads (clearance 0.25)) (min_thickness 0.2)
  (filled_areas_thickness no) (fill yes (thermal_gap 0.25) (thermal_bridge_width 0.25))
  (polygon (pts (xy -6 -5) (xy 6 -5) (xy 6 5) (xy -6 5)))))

